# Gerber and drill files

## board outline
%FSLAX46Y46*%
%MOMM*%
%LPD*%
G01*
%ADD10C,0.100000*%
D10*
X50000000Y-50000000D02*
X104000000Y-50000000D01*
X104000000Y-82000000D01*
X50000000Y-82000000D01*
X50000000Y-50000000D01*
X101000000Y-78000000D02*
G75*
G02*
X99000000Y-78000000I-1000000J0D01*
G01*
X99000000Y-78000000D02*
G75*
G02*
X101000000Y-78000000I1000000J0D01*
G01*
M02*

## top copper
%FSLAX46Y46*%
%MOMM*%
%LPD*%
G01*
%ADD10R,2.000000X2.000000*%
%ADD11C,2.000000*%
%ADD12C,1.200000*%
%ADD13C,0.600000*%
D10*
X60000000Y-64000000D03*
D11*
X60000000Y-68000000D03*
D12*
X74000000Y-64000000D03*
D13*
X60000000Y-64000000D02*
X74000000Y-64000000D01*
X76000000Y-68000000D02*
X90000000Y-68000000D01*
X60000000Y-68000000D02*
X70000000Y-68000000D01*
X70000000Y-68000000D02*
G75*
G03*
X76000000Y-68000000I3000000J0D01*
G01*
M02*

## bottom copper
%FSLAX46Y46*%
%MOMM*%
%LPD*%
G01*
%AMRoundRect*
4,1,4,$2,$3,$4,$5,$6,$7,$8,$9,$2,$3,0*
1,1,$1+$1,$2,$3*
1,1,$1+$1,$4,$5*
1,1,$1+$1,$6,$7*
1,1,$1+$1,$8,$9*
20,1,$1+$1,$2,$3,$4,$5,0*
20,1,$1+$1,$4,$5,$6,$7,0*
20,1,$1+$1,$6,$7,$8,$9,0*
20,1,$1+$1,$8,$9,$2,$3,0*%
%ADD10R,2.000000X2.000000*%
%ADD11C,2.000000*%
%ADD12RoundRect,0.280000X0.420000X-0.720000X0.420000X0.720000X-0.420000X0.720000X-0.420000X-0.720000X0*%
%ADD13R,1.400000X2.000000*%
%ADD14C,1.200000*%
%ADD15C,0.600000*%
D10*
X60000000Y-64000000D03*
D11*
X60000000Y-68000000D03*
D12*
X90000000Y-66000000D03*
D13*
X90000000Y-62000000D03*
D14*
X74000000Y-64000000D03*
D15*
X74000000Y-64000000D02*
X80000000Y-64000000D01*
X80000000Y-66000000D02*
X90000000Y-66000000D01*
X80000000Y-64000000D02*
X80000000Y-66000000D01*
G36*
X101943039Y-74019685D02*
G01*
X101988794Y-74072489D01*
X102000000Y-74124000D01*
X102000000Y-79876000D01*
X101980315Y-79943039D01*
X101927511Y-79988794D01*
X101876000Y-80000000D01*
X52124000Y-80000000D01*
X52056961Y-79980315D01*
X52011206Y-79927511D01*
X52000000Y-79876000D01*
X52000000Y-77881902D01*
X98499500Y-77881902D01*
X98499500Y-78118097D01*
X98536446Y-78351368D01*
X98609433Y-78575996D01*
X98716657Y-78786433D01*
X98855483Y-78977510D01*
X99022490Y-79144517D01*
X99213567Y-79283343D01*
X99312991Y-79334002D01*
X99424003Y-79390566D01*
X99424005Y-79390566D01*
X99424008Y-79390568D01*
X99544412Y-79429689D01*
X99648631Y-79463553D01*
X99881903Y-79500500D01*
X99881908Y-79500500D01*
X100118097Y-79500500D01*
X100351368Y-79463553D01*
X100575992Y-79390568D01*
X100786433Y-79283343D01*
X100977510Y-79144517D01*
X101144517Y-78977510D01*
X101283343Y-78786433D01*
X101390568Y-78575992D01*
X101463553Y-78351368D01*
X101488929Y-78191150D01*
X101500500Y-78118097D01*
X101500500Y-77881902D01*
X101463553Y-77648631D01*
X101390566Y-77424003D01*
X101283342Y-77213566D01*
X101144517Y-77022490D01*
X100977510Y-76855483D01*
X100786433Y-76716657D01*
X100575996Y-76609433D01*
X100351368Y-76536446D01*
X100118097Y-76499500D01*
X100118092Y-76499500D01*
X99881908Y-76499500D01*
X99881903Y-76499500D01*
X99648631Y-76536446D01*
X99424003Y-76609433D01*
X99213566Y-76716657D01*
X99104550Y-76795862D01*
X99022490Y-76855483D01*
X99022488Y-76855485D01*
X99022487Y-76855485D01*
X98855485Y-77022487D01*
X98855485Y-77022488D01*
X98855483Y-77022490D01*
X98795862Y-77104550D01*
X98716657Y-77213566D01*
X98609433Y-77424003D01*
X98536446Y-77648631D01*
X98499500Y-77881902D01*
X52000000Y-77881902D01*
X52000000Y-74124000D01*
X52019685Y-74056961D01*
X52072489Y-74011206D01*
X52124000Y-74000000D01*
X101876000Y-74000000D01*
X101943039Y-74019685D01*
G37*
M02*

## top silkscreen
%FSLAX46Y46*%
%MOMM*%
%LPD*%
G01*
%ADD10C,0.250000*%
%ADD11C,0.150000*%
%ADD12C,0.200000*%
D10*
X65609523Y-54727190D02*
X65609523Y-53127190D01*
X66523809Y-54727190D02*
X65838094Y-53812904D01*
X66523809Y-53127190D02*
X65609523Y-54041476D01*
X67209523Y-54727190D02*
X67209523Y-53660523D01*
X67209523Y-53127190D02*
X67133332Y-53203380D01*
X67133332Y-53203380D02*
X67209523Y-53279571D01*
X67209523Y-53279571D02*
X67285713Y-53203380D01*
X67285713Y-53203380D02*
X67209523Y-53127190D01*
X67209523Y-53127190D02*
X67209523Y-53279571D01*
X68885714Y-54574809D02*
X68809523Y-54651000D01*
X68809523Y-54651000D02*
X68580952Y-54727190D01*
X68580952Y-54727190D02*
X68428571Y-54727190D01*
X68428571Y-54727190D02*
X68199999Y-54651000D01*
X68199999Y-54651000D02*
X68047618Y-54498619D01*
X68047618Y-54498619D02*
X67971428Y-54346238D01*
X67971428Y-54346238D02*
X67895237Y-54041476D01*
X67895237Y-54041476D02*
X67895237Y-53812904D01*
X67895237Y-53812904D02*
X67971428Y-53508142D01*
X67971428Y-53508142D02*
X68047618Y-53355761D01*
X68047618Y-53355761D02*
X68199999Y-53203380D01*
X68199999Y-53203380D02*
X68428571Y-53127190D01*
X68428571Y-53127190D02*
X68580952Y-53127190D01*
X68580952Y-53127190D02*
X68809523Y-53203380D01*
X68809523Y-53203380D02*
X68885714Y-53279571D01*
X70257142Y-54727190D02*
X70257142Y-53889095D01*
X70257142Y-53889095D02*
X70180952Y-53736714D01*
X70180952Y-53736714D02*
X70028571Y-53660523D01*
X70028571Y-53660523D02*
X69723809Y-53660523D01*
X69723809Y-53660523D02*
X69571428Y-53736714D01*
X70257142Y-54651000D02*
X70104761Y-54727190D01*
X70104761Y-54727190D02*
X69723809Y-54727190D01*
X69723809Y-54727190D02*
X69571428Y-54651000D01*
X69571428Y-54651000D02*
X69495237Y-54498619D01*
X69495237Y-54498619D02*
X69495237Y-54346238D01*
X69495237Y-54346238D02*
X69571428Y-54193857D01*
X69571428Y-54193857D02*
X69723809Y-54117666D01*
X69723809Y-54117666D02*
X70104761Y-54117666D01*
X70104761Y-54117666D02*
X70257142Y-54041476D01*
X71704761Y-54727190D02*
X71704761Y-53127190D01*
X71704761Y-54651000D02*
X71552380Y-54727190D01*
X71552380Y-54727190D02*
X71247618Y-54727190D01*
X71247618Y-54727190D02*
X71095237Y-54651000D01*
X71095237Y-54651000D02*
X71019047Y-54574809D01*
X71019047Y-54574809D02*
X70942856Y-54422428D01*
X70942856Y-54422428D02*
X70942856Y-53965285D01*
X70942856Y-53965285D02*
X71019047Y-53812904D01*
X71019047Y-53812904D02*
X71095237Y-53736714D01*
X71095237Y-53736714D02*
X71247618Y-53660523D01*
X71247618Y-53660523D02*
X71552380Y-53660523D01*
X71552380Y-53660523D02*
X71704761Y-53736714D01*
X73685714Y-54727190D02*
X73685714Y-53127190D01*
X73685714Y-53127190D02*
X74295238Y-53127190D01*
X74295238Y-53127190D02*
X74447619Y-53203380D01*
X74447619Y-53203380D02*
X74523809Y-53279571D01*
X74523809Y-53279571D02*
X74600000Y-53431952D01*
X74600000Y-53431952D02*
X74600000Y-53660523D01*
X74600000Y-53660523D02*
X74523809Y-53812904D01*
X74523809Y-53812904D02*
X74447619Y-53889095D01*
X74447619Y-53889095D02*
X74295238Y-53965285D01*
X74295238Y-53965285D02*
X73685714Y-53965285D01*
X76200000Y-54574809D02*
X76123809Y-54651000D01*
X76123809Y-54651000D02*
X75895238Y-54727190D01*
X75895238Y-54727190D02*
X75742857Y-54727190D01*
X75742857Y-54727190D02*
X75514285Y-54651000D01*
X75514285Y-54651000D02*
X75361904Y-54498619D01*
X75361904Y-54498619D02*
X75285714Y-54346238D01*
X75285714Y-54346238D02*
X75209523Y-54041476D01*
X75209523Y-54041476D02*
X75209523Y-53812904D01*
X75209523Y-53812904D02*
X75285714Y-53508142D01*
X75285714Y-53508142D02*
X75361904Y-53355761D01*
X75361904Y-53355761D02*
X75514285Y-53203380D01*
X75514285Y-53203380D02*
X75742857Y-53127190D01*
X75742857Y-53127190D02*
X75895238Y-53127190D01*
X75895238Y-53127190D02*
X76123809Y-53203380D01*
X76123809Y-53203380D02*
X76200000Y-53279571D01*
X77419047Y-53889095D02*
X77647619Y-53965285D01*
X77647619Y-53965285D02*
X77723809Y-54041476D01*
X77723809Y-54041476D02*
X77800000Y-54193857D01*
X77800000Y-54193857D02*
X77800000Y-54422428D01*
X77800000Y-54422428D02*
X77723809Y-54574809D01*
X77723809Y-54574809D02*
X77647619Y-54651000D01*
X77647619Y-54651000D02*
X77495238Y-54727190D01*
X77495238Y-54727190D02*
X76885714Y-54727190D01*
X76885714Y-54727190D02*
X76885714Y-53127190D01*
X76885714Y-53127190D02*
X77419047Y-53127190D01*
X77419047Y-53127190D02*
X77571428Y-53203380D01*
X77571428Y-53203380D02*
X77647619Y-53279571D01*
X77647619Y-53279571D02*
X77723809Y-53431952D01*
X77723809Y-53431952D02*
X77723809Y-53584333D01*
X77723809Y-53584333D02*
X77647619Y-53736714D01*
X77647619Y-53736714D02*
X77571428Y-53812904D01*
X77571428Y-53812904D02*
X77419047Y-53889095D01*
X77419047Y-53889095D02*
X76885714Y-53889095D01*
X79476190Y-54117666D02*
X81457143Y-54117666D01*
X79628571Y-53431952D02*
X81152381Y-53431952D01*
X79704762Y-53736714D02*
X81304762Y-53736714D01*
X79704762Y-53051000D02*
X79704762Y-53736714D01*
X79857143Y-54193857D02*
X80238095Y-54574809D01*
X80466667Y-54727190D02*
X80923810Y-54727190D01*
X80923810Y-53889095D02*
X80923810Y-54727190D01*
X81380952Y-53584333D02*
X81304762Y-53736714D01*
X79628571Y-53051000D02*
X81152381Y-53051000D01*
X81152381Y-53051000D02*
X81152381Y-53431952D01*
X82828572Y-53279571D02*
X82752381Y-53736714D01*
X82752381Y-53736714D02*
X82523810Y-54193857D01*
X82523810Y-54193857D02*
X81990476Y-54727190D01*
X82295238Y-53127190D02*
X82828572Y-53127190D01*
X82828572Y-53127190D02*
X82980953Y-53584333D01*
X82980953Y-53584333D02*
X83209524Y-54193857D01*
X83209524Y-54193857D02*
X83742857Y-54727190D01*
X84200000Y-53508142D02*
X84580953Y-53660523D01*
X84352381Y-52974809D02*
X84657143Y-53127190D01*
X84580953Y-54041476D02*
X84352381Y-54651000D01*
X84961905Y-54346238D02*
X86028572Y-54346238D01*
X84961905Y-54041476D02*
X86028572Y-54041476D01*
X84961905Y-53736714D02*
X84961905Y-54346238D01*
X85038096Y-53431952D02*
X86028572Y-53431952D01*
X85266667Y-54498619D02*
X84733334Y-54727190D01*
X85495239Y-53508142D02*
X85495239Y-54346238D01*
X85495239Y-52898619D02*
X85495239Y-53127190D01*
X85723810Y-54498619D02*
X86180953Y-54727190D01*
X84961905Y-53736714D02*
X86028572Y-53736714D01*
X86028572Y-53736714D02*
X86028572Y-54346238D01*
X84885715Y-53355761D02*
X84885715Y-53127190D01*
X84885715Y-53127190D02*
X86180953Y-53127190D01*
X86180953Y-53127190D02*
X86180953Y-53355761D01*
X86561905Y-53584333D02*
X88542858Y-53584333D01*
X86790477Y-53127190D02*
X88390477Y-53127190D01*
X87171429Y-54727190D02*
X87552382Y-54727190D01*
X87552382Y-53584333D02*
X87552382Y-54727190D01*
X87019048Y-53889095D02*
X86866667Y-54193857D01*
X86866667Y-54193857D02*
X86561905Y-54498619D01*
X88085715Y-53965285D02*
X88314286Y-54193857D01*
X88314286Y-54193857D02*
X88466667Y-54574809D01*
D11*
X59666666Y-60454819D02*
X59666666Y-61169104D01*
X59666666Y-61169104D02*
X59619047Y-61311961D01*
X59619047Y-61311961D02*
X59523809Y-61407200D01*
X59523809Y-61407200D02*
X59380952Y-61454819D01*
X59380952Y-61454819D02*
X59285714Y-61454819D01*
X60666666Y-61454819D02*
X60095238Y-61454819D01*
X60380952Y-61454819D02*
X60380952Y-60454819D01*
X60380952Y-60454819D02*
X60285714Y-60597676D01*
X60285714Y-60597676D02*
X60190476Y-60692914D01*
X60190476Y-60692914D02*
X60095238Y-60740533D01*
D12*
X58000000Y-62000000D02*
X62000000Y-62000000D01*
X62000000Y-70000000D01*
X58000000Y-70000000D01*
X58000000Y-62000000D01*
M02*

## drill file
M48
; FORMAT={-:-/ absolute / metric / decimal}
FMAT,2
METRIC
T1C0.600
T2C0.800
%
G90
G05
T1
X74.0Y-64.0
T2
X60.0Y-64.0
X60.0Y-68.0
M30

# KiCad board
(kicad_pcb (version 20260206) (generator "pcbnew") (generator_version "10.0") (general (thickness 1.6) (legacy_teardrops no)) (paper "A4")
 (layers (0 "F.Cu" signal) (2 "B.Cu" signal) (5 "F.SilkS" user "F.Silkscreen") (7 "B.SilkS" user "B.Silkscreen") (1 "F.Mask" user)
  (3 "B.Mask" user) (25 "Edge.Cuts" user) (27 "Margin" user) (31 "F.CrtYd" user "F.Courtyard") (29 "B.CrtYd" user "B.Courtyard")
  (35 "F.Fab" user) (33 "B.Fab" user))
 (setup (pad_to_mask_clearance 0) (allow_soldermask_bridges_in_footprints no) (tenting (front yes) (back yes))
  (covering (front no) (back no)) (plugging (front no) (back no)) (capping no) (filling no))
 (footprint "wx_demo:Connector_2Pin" (layer "F.Cu") (at 60 64)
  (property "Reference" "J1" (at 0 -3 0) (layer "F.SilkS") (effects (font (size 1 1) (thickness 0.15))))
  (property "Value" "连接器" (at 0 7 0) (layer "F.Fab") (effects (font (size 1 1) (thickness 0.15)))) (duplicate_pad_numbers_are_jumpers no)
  (fp_rect (start -2 -2) (end 2 6) (stroke (width 0.2) (type solid)) (fill no) (layer "F.SilkS"))
  (pad "1" thru_hole rect (at 0 0) (size 2 2) (drill 0.8) (layers "*.Cu" "*.Mask") (remove_unused_layers no) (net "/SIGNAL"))
  (pad "2" thru_hole circle (at 0 4) (size 2 2) (drill 0.8) (layers "*.Cu" "*.Mask") (remove_unused_layers no) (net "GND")))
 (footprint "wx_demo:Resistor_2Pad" (layer "B.Cu") (at 90 64 90)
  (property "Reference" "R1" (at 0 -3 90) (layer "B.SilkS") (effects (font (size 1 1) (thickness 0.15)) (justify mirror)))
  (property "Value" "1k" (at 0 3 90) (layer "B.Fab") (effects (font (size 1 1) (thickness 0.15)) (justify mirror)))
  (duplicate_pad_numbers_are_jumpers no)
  (pad "1" smd roundrect (at -2 0 90) (size 2 1.4) (layers "B.Cu" "B.Mask") (roundrect_rratio 0.2) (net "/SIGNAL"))
  (pad "2" smd rect (at 2 0 90) (size 2 1.4) (layers "B.Cu" "B.Mask") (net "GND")))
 (gr_rect (start 50 50) (end 104 82) (stroke (width 0.1) (type solid)) (fill no) (layer "Edge.Cuts"))
 (gr_circle (center 100 78) (end 101 78) (stroke (width 0.1) (type solid)) (fill no) (layer "Edge.Cuts"))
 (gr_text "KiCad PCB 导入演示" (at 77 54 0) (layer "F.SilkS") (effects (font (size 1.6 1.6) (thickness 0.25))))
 (segment (start 60 64) (end 74 64) (width 0.6) (layer "F.Cu") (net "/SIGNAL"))
 (via (at 74 64) (size 1.2) (drill 0.6) (layers "F.Cu" "B.Cu") (capping no) (covering (front no) (back no)) (plugging (front no) (back no))
  (filling no) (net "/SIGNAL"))
 (segment (start 74 64) (end 80 64) (width 0.6) (layer "B.Cu") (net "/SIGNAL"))
 (segment (start 80 66) (end 90 66) (width 0.6) (layer "B.Cu") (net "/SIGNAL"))
 (segment (start 80 64) (end 80 66) (width 0.6) (layer "B.Cu") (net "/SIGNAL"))
 (segment (start 76 68) (end 90 68) (width 0.6) (layer "F.Cu") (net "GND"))
 (segment (start 60 68) (end 70 68) (width 0.6) (layer "F.Cu") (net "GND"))
 (arc (start 70 68) (mid 73 71) (end 76 68) (width 0.6) (layer "F.Cu") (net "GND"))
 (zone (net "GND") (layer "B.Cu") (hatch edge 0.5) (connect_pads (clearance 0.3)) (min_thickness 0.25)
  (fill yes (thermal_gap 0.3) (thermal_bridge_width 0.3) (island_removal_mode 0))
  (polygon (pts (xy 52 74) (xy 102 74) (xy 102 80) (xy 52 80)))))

